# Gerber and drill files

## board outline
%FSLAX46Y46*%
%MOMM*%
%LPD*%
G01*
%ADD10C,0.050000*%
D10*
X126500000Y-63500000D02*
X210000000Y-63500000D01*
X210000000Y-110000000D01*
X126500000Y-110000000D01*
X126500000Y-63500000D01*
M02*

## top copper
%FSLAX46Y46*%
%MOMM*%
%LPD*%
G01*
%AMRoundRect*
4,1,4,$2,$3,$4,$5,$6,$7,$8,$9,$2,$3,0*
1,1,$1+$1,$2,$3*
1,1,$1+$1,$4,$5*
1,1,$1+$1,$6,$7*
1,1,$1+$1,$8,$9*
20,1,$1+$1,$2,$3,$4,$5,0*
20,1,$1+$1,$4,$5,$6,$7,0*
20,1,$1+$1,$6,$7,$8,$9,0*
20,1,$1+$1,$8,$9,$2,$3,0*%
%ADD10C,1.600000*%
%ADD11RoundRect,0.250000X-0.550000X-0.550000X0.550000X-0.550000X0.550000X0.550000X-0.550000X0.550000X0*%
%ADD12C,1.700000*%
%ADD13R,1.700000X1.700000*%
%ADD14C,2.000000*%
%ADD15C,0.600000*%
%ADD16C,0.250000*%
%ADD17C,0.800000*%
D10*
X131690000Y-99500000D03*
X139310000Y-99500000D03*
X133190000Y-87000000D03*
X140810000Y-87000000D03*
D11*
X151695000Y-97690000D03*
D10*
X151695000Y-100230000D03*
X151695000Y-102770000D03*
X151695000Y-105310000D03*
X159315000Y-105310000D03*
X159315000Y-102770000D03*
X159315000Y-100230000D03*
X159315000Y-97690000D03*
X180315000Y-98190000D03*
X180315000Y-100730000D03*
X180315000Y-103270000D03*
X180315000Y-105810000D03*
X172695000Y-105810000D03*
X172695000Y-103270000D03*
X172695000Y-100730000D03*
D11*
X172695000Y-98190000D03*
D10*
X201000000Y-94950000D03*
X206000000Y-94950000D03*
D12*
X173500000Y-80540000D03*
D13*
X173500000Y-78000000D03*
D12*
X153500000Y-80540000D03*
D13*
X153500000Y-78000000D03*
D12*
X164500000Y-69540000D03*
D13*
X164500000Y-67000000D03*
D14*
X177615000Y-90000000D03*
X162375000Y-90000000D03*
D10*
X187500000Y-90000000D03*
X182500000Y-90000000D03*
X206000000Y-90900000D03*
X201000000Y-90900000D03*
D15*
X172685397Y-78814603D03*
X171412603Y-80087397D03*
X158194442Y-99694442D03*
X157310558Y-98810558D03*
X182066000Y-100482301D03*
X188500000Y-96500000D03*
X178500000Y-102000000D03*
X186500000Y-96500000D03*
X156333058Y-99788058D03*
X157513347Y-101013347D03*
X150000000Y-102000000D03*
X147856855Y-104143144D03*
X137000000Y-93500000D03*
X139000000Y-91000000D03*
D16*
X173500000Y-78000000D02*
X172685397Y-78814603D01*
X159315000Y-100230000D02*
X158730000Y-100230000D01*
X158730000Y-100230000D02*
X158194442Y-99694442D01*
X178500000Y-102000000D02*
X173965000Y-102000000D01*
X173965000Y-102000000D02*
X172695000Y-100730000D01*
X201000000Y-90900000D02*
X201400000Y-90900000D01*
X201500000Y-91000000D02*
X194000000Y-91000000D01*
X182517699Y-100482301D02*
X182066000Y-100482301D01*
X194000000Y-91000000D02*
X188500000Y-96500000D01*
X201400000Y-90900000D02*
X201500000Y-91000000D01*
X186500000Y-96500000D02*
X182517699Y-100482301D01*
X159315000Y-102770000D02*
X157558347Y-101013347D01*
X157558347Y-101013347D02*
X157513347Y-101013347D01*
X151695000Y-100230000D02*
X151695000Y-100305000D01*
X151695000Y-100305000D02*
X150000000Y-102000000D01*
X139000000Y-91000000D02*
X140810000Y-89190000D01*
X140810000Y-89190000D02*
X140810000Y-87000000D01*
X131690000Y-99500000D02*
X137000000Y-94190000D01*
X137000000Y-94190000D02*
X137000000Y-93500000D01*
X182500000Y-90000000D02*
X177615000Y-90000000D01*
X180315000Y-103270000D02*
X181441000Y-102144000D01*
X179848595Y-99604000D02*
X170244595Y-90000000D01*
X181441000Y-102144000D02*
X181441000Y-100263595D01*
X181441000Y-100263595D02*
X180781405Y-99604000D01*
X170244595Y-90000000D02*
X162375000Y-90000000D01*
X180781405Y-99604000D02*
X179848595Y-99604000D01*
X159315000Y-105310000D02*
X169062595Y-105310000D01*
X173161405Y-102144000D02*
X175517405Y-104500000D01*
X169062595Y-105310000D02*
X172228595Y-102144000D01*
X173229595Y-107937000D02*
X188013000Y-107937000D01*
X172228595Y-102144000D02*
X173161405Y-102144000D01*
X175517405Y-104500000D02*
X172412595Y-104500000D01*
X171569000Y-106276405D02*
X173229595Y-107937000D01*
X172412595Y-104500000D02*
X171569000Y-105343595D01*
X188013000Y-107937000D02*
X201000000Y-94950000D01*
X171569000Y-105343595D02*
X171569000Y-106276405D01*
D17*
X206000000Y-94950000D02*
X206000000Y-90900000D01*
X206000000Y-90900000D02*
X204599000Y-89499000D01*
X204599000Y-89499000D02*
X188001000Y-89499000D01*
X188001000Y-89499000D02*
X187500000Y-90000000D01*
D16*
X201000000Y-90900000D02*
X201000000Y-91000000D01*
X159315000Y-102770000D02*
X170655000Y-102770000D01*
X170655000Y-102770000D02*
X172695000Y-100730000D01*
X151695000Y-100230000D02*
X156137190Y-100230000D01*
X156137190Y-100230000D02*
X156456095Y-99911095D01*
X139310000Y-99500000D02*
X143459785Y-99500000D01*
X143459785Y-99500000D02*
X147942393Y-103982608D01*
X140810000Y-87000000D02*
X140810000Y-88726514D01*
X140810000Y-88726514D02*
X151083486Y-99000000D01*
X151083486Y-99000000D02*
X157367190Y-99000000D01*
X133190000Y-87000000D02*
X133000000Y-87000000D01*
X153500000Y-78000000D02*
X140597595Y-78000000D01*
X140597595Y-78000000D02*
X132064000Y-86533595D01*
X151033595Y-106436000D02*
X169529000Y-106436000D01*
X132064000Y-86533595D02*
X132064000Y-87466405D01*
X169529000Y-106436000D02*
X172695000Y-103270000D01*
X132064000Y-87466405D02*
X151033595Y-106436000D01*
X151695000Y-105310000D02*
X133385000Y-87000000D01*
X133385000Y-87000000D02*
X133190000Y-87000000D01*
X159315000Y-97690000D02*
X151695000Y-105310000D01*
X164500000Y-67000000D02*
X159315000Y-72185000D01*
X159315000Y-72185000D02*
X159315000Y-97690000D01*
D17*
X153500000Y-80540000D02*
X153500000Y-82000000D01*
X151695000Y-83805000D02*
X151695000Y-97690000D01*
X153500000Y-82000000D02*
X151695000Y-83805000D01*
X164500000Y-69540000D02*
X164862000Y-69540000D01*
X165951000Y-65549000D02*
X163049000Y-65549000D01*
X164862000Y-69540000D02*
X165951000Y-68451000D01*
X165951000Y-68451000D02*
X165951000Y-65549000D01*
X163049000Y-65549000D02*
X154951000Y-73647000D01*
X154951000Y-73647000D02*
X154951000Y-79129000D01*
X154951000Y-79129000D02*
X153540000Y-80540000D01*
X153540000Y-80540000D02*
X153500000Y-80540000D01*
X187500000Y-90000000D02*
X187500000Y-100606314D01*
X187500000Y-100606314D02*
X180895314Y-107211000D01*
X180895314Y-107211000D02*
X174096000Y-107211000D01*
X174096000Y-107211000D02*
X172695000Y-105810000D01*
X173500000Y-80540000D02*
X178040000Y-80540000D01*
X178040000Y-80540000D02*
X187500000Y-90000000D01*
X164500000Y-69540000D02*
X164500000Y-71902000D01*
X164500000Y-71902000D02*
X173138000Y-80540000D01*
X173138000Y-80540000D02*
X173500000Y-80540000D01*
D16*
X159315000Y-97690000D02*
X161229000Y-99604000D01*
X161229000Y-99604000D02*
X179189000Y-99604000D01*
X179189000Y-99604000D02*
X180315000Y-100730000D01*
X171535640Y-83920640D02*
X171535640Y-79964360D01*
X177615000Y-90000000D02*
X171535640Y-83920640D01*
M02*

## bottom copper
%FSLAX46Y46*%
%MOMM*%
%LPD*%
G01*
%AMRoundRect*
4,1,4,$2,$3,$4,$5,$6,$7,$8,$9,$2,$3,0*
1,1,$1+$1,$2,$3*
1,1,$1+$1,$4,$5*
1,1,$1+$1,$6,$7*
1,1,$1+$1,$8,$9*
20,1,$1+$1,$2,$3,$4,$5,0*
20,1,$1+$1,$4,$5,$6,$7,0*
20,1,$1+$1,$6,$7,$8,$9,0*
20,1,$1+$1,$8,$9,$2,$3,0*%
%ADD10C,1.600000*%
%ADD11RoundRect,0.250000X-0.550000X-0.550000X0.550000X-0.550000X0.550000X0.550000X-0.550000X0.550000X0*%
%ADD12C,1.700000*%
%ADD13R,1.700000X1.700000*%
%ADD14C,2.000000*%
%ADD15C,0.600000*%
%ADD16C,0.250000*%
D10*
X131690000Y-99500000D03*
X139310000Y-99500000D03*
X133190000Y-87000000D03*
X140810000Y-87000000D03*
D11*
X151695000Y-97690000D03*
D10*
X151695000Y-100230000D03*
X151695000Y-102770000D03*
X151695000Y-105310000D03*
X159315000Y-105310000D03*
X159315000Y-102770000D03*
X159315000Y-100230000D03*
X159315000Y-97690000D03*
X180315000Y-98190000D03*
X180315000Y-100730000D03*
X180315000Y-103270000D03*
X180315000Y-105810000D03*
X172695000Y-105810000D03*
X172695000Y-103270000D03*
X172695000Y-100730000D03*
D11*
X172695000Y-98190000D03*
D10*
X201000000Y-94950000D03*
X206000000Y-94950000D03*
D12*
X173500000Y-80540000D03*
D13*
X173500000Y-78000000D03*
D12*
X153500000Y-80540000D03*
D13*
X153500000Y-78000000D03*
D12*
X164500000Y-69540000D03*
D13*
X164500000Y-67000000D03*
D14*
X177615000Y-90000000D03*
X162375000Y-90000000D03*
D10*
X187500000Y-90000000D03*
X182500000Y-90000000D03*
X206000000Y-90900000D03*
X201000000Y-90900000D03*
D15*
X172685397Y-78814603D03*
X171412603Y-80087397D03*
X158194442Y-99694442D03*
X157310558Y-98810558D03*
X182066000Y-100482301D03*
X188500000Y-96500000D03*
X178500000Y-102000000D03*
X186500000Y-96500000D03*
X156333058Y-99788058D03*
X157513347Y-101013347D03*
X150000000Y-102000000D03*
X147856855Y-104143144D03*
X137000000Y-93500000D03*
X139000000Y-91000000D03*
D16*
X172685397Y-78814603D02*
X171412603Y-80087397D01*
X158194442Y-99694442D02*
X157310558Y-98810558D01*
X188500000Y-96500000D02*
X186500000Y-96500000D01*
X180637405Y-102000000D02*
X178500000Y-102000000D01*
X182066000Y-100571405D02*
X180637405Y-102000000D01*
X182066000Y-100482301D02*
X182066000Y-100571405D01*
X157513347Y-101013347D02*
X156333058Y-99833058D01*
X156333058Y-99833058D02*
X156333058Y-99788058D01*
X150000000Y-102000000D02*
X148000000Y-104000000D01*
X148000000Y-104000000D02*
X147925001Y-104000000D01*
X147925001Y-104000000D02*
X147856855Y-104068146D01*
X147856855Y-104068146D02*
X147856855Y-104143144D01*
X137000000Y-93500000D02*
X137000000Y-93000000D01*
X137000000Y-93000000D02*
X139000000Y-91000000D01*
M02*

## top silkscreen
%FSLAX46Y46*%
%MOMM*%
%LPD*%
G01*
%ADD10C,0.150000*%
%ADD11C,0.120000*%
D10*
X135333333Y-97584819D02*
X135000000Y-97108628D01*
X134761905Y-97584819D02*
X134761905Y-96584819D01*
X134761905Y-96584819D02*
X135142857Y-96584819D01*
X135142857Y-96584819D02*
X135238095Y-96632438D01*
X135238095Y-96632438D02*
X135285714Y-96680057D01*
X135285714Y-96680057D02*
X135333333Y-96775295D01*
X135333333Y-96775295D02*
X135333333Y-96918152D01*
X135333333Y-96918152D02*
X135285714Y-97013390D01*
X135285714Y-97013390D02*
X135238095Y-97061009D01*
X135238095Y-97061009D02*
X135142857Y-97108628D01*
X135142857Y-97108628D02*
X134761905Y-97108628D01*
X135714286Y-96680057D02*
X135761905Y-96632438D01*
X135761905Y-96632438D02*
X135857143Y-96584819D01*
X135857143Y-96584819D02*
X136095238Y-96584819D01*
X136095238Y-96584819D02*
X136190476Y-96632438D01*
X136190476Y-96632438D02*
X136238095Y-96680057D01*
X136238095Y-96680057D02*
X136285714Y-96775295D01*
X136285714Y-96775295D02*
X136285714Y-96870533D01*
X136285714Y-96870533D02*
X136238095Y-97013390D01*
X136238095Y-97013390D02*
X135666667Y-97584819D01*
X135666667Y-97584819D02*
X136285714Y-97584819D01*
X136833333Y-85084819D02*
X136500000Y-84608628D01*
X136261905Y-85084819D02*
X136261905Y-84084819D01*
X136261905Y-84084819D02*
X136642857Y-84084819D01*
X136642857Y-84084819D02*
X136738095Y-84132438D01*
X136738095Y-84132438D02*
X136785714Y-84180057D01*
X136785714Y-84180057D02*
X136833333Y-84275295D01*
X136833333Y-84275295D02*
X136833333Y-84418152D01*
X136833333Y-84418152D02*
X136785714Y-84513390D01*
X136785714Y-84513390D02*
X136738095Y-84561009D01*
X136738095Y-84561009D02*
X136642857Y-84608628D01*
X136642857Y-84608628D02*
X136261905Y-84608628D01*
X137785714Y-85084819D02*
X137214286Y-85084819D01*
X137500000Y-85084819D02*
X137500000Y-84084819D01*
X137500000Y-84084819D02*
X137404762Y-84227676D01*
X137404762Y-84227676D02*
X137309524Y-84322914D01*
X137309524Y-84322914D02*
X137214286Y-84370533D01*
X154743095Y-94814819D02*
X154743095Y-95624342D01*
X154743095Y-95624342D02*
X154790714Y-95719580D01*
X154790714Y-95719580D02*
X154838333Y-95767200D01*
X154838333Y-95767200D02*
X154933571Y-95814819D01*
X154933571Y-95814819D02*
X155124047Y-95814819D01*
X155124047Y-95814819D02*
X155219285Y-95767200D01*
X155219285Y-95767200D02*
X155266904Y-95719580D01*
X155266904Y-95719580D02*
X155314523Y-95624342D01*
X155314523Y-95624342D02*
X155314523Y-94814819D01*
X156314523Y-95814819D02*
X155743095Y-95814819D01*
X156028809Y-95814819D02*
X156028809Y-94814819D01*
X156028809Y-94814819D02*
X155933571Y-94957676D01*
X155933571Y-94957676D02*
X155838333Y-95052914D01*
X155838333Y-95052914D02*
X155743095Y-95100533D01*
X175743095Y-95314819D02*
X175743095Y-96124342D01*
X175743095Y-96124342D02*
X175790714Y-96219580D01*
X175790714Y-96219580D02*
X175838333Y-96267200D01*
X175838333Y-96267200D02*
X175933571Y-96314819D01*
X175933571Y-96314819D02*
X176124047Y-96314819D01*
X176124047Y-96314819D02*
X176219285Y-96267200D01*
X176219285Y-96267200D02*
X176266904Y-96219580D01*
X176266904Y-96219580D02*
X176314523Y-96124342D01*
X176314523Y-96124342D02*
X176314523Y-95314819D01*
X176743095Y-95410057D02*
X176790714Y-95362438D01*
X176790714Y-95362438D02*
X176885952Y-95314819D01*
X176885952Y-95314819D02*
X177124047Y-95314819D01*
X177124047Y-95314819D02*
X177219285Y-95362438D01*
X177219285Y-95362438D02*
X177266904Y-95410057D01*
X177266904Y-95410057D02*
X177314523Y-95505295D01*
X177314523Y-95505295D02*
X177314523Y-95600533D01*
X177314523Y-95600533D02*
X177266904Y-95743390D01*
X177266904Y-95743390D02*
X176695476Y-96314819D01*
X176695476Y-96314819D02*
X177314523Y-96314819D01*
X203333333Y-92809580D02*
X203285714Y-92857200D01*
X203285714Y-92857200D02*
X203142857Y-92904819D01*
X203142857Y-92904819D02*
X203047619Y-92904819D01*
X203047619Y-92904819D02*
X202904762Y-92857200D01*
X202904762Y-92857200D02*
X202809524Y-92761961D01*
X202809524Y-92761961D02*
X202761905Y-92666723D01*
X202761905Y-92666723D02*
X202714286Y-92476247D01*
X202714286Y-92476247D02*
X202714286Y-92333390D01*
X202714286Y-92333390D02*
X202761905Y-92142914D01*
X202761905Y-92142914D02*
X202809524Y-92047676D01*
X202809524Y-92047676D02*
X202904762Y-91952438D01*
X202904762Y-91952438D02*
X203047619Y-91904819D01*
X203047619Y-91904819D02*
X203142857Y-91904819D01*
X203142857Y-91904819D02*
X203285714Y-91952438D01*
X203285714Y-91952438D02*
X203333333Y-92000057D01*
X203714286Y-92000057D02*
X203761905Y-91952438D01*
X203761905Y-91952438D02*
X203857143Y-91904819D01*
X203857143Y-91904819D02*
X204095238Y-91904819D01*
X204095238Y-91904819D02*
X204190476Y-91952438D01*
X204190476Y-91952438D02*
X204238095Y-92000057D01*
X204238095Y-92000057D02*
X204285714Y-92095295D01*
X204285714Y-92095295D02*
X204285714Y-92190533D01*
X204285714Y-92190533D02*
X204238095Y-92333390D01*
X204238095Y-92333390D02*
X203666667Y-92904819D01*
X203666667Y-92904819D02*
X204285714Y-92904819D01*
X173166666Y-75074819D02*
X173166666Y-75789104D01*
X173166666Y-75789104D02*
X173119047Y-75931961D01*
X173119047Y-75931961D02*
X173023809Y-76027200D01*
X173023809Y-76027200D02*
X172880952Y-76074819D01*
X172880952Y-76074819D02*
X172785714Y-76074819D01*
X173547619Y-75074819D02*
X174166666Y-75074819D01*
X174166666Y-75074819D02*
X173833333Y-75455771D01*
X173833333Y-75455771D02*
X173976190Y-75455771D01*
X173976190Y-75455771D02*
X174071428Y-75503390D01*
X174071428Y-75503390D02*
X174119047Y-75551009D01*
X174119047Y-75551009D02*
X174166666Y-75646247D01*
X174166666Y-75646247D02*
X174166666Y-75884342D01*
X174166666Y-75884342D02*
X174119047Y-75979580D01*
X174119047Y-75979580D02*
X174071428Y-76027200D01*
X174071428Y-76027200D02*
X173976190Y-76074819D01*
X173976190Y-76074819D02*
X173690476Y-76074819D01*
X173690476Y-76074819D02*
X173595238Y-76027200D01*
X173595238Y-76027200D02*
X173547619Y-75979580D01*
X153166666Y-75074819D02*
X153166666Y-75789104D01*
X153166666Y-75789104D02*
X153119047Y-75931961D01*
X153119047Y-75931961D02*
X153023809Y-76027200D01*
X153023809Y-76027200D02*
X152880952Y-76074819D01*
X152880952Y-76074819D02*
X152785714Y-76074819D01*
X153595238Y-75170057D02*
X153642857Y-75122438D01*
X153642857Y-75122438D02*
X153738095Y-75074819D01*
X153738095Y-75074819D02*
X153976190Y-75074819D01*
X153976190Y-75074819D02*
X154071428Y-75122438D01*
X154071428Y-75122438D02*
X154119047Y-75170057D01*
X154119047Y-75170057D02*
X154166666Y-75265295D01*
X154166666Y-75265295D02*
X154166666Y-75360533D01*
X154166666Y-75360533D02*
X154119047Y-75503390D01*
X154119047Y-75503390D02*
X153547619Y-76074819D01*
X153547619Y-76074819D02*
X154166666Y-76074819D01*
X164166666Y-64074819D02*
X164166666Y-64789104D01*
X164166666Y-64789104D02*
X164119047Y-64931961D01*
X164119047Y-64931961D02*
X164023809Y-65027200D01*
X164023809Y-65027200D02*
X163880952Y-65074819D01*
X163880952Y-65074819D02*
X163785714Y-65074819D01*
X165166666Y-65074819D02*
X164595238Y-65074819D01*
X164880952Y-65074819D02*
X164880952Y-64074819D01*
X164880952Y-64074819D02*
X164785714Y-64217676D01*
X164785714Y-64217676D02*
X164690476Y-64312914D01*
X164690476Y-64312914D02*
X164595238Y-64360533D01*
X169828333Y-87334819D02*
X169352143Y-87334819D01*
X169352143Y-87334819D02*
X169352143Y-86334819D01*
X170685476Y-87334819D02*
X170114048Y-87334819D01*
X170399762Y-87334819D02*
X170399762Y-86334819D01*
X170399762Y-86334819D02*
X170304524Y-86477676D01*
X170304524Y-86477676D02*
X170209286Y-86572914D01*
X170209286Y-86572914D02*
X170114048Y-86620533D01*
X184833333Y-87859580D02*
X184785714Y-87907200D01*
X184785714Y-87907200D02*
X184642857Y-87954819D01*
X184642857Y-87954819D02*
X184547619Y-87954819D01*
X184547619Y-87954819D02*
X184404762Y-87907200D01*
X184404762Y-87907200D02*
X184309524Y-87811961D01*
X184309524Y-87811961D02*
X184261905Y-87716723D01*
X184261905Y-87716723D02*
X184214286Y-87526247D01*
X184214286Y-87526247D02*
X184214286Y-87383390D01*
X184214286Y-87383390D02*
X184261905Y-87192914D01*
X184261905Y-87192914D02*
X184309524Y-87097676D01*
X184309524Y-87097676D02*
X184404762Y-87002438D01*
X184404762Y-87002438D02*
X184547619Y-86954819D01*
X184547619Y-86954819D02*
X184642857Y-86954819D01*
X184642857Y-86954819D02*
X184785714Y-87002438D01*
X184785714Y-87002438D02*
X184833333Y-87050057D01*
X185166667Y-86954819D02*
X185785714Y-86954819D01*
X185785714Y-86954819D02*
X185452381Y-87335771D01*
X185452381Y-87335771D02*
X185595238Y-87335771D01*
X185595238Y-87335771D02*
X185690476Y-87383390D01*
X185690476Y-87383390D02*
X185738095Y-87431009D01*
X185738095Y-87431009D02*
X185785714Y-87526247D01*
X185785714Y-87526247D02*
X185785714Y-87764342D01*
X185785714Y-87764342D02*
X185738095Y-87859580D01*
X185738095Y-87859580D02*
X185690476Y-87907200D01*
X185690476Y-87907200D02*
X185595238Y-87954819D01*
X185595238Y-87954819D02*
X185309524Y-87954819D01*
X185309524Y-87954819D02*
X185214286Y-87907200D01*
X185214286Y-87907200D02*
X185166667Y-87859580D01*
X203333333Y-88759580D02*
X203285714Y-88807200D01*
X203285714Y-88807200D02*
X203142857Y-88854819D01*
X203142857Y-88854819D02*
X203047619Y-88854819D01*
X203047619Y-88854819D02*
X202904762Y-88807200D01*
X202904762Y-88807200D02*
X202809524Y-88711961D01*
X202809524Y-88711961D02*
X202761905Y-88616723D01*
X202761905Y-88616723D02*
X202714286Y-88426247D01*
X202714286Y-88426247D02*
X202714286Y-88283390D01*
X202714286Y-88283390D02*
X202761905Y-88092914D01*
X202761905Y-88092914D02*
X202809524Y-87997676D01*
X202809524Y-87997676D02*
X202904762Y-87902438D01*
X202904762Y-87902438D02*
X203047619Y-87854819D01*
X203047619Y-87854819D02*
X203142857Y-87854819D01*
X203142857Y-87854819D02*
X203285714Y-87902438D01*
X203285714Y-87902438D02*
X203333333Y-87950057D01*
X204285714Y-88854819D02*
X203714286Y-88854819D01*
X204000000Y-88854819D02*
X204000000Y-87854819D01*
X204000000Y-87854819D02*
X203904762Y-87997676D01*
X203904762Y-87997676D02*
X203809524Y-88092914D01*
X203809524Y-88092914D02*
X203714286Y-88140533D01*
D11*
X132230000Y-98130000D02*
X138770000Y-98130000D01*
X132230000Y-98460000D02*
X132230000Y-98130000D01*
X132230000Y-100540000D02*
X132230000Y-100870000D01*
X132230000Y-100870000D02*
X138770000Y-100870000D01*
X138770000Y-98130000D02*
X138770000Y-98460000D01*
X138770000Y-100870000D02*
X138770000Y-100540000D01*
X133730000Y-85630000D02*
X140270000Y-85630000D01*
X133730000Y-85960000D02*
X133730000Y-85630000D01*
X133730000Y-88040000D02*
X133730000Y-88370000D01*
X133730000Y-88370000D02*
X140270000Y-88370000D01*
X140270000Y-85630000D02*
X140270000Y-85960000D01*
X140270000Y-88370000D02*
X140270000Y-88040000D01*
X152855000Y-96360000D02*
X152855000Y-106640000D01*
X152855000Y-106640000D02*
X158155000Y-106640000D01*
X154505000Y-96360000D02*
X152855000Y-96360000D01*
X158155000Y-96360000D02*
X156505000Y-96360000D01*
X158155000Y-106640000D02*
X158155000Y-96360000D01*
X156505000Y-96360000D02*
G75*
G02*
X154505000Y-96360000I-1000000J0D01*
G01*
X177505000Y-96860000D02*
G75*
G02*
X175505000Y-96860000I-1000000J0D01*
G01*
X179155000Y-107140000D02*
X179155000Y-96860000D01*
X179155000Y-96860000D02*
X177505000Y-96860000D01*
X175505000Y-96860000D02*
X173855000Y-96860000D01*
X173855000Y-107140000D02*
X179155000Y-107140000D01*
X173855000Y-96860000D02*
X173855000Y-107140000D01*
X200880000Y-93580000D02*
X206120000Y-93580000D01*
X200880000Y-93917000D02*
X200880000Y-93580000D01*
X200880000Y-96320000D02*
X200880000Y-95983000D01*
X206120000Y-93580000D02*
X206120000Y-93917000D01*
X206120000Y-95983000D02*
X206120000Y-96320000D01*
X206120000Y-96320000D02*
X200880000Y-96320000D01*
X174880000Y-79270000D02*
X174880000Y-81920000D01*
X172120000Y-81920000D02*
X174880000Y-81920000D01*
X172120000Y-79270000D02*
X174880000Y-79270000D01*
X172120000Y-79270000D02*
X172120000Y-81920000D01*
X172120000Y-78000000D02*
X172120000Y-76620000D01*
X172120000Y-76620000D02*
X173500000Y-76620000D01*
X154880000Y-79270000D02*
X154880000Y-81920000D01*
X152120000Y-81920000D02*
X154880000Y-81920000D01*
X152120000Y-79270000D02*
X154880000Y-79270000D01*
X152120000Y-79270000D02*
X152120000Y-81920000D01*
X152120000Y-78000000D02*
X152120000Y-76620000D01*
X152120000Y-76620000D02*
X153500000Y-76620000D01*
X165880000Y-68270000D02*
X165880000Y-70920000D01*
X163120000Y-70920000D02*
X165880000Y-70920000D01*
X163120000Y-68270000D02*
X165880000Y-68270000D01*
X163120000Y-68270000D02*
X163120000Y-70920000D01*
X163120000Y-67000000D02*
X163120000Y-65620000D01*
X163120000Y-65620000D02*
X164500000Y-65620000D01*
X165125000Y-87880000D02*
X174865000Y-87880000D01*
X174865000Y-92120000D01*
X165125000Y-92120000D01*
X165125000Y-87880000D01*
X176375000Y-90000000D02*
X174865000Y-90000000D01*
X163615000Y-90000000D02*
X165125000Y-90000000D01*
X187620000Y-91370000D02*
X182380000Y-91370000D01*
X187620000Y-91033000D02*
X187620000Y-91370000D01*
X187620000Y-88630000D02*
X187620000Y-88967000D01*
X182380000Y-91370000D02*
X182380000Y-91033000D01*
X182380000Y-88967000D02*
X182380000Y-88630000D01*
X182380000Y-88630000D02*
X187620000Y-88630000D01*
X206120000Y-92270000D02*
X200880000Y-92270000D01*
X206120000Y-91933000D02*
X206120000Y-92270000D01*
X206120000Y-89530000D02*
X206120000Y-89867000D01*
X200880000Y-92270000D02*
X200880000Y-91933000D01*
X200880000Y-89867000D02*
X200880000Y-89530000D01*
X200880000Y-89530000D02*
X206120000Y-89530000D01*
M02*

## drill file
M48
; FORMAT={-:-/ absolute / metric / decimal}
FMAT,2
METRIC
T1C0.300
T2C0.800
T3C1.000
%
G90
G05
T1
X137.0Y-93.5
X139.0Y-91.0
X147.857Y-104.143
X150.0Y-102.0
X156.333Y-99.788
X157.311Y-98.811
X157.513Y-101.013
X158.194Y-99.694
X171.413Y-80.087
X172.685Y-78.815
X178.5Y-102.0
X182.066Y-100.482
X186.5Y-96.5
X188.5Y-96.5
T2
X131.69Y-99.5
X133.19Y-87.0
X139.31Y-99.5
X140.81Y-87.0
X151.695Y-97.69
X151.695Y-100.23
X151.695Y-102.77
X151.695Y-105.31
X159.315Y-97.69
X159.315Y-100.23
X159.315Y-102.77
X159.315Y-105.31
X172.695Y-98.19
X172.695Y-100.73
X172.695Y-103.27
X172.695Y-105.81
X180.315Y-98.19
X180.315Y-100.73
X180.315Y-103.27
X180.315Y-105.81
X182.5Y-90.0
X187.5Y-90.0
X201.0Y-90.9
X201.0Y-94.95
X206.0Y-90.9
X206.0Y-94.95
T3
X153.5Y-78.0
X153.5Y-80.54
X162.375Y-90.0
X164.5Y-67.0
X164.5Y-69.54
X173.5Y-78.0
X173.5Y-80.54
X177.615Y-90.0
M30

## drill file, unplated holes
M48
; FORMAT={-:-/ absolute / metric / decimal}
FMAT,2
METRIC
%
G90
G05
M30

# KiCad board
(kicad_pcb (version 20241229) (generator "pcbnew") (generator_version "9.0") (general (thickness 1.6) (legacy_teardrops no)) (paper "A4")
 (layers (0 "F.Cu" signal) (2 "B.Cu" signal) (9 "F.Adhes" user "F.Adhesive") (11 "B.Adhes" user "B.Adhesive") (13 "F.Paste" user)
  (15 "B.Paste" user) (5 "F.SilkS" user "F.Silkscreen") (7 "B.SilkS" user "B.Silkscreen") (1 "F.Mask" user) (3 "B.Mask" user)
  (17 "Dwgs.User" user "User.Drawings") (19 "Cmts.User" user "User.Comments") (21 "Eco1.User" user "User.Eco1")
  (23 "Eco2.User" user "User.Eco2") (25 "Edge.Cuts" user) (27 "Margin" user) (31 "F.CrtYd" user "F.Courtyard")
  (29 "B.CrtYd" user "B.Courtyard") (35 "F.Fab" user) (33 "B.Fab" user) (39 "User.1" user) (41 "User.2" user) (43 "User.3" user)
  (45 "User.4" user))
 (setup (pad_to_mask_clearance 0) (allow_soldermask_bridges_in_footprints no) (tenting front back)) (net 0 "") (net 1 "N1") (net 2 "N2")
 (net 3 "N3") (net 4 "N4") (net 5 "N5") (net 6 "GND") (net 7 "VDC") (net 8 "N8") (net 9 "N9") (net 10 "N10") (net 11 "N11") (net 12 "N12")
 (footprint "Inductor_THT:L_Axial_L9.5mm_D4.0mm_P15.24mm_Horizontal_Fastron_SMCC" (layer "F.Cu") (at 162.375 90)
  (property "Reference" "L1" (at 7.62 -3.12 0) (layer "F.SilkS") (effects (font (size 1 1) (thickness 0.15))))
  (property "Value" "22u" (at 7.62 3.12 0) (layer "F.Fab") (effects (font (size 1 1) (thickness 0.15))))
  (fp_line (start 1.24 0) (end 2.75 0) (stroke (width 0.12) (type solid)) (layer "F.SilkS"))
  (fp_line (start 14 0) (end 12.49 0) (stroke (width 0.12) (type solid)) (layer "F.SilkS"))
  (fp_rect (start 2.75 -2.12) (end 12.49 2.12) (stroke (width 0.12) (type solid)) (fill no) (layer "F.SilkS"))
  (pad "1" thru_hole circle (at 0 0) (size 2 2) (drill 1) (layers "*.Cu" "*.Mask") (remove_unused_layers no) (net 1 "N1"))
  (pad "2" thru_hole circle (at 15.24 0) (size 2 2) (drill 1) (layers "*.Cu" "*.Mask") (remove_unused_layers no) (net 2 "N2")))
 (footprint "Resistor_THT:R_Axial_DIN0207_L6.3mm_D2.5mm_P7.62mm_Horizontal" (layer "F.Cu") (at 131.69 99.5)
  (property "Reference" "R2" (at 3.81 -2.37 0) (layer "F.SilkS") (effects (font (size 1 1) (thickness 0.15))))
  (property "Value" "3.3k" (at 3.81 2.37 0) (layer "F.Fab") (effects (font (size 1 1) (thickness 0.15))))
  (fp_line (start 0.54 -1.37) (end 7.08 -1.37) (stroke (width 0.12) (type solid)) (layer "F.SilkS"))
  (fp_line (start 0.54 -1.04) (end 0.54 -1.37) (stroke (width 0.12) (type solid)) (layer "F.SilkS"))
  (fp_line (start 0.54 1.04) (end 0.54 1.37) (stroke (width 0.12) (type solid)) (layer "F.SilkS"))
  (fp_line (start 0.54 1.37) (end 7.08 1.37) (stroke (width 0.12) (type solid)) (layer "F.SilkS"))
  (fp_line (start 7.08 -1.37) (end 7.08 -1.04) (stroke (width 0.12) (type solid)) (layer "F.SilkS"))
  (fp_line (start 7.08 1.37) (end 7.08 1.04) (stroke (width 0.12) (type solid)) (layer "F.SilkS"))
  (pad "1" thru_hole circle (at 0 0) (size 1.6 1.6) (drill 0.8) (layers "*.Cu" "*.Mask") (remove_unused_layers no) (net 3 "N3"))
  (pad "2" thru_hole circle (at 7.62 0) (size 1.6 1.6) (drill 0.8) (layers "*.Cu" "*.Mask") (remove_unused_layers no) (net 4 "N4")))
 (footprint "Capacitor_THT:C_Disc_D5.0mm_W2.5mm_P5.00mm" (layer "F.Cu") (at 201 94.95)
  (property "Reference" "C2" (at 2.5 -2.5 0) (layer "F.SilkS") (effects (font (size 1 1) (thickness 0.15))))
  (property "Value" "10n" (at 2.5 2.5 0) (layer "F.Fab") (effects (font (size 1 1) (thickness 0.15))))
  (fp_line (start -0.12 -1.37) (end 5.12 -1.37) (stroke (width 0.12) (type solid)) (layer "F.SilkS"))
  (fp_line (start -0.12 -1.033) (end -0.12 -1.37) (stroke (width 0.12) (type solid)) (layer "F.SilkS"))
  (fp_line (start -0.12 1.37) (end -0.12 1.033) (stroke (width 0.12) (type solid)) (layer "F.SilkS"))
  (fp_line (start 5.12 -1.37) (end 5.12 -1.033) (stroke (width 0.12) (type solid)) (layer "F.SilkS"))
  (fp_line (start 5.12 1.033) (end 5.12 1.37) (stroke (width 0.12) (type solid)) (layer "F.SilkS"))
  (fp_line (start 5.12 1.37) (end -0.12 1.37) (stroke (width 0.12) (type solid)) (layer "F.SilkS"))
  (pad "1" thru_hole circle (at 0 0) (size 1.6 1.6) (drill 0.8) (layers "*.Cu" "*.Mask") (remove_unused_layers no) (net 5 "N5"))
  (pad "2" thru_hole circle (at 5 0) (size 1.6 1.6) (drill 0.8) (layers "*.Cu" "*.Mask") (remove_unused_layers no) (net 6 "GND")))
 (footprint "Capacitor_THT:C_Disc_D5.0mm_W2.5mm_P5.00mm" (layer "F.Cu") (at 182.5 90)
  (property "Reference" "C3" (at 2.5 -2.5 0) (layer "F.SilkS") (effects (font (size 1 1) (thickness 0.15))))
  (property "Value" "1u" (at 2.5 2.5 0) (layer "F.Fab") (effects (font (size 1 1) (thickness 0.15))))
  (fp_line (start -0.12 -1.37) (end 5.12 -1.37) (stroke (width 0.12) (type solid)) (layer "F.SilkS"))
  (fp_line (start -0.12 -1.033) (end -0.12 -1.37) (stroke (width 0.12) (type solid)) (layer "F.SilkS"))
  (fp_line (start -0.12 1.37) (end -0.12 1.033) (stroke (width 0.12) (type solid)) (layer "F.SilkS"))
  (fp_line (start 5.12 -1.37) (end 5.12 -1.033) (stroke (width 0.12) (type solid)) (layer "F.SilkS"))
  (fp_line (start 5.12 1.033) (end 5.12 1.37) (stroke (width 0.12) (type solid)) (layer "F.SilkS"))
  (fp_line (start 5.12 1.37) (end -0.12 1.37) (stroke (width 0.12) (type solid)) (layer "F.SilkS"))
  (pad "1" thru_hole circle (at 0 0) (size 1.6 1.6) (drill 0.8) (layers "*.Cu" "*.Mask") (remove_unused_layers no) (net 2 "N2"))
  (pad "2" thru_hole circle (at 5 0) (size 1.6 1.6) (drill 0.8) (layers "*.Cu" "*.Mask") (remove_unused_layers no) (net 6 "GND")))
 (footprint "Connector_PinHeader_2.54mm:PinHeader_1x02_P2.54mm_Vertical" (layer "F.Cu") (at 164.5 67)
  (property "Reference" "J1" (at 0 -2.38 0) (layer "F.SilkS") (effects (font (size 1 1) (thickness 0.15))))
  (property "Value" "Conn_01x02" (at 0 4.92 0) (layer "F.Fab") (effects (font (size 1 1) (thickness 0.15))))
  (fp_line (start -1.38 -1.38) (end 0 -1.38) (stroke (width 0.12) (type solid)) (layer "F.SilkS"))
  (fp_line (start -1.38 0) (end -1.38 -1.38) (stroke (width 0.12) (type solid)) (layer "F.SilkS"))
  (fp_line (start -1.38 1.27) (end -1.38 3.92) (stroke (width 0.12) (type solid)) (layer "F.SilkS"))
  (fp_line (start -1.38 1.27) (end 1.38 1.27) (stroke (width 0.12) (type solid)) (layer "F.SilkS"))
  (fp_line (start -1.38 3.92) (end 1.38 3.92) (stroke (width 0.12) (type solid)) (layer "F.SilkS"))
  (fp_line (start 1.38 1.27) (end 1.38 3.92) (stroke (width 0.12) (type solid)) (layer "F.SilkS"))
  (pad "1" thru_hole rect (at 0 0) (size 1.7 1.7) (drill 1) (layers "*.Cu" "*.Mask") (remove_unused_layers no) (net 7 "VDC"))
  (pad "2" thru_hole circle (at 0 2.54) (size 1.7 1.7) (drill 1) (layers "*.Cu" "*.Mask") (remove_unused_layers no) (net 6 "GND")))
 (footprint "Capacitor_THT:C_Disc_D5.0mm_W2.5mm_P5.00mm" (layer "F.Cu") (at 201 90.9)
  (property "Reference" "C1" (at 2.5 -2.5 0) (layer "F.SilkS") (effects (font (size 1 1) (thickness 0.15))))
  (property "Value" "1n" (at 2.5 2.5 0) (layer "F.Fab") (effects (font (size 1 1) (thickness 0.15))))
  (fp_line (start -0.12 -1.37) (end 5.12 -1.37) (stroke (width 0.12) (type solid)) (layer "F.SilkS"))
  (fp_line (start -0.12 -1.033) (end -0.12 -1.37) (stroke (width 0.12) (type solid)) (layer "F.SilkS"))
  (fp_line (start -0.12 1.37) (end -0.12 1.033) (stroke (width 0.12) (type solid)) (layer "F.SilkS"))
  (fp_line (start 5.12 -1.37) (end 5.12 -1.033) (stroke (width 0.12) (type solid)) (layer "F.SilkS"))
  (fp_line (start 5.12 1.033) (end 5.12 1.37) (stroke (width 0.12) (type solid)) (layer "F.SilkS"))
  (fp_line (start 5.12 1.37) (end -0.12 1.37) (stroke (width 0.12) (type solid)) (layer "F.SilkS"))
  (pad "1" thru_hole circle (at 0 0) (size 1.6 1.6) (drill 0.8) (layers "*.Cu" "*.Mask") (remove_unused_layers no) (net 4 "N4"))
  (pad "2" thru_hole circle (at 5 0) (size 1.6 1.6) (drill 0.8) (layers "*.Cu" "*.Mask") (remove_unused_layers no) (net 6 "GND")))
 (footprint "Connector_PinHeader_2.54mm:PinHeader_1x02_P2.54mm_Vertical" (layer "F.Cu") (at 153.5 78)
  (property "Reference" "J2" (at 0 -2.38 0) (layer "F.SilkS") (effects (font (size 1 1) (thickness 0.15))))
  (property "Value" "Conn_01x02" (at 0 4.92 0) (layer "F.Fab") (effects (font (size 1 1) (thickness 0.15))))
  (fp_line (start -1.38 -1.38) (end 0 -1.38) (stroke (width 0.12) (type solid)) (layer "F.SilkS"))
  (fp_line (start -1.38 0) (end -1.38 -1.38) (stroke (width 0.12) (type solid)) (layer "F.SilkS"))
  (fp_line (start -1.38 1.27) (end -1.38 3.92) (stroke (width 0.12) (type solid)) (layer "F.SilkS"))
  (fp_line (start -1.38 1.27) (end 1.38 1.27) (stroke (width 0.12) (type solid)) (layer "F.SilkS"))
  (fp_line (start -1.38 3.92) (end 1.38 3.92) (stroke (width 0.12) (type solid)) (layer "F.SilkS"))
  (fp_line (start 1.38 1.27) (end 1.38 3.92) (stroke (width 0.12) (type solid)) (layer "F.SilkS"))
  (pad "1" thru_hole rect (at 0 0) (size 1.7 1.7) (drill 1) (layers "*.Cu" "*.Mask") (remove_unused_layers no) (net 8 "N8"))
  (pad "2" thru_hole circle (at 0 2.54) (size 1.7 1.7) (drill 1) (layers "*.Cu" "*.Mask") (remove_unused_layers no) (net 6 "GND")))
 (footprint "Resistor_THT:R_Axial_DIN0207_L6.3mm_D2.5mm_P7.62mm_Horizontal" (layer "F.Cu") (at 133.19 87)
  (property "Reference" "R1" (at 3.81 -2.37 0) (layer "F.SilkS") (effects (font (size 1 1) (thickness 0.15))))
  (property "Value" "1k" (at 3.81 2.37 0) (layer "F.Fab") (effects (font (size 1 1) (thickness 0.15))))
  (fp_line (start 0.54 -1.37) (end 7.08 -1.37) (stroke (width 0.12) (type solid)) (layer "F.SilkS"))
  (fp_line (start 0.54 -1.04) (end 0.54 -1.37) (stroke (width 0.12) (type solid)) (layer "F.SilkS"))
  (fp_line (start 0.54 1.04) (end 0.54 1.37) (stroke (width 0.12) (type solid)) (layer "F.SilkS"))
  (fp_line (start 0.54 1.37) (end 7.08 1.37) (stroke (width 0.12) (type solid)) (layer "F.SilkS"))
  (fp_line (start 7.08 -1.37) (end 7.08 -1.04) (stroke (width 0.12) (type solid)) (layer "F.SilkS"))
  (fp_line (start 7.08 1.37) (end 7.08 1.04) (stroke (width 0.12) (type solid)) (layer "F.SilkS"))
  (pad "1" thru_hole circle (at 0 0) (size 1.6 1.6) (drill 0.8) (layers "*.Cu" "*.Mask") (remove_unused_layers no) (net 7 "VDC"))
  (pad "2" thru_hole circle (at 7.62 0) (size 1.6 1.6) (drill 0.8) (layers "*.Cu" "*.Mask") (remove_unused_layers no) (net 3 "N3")))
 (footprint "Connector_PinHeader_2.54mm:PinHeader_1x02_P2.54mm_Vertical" (layer "F.Cu") (at 173.5 78)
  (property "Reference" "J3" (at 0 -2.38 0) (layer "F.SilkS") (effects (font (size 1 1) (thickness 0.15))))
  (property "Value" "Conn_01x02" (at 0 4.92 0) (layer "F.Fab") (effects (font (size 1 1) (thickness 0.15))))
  (fp_line (start -1.38 -1.38) (end 0 -1.38) (stroke (width 0.12) (type solid)) (layer "F.SilkS"))
  (fp_line (start -1.38 0) (end -1.38 -1.38) (stroke (width 0.12) (type solid)) (layer "F.SilkS"))
  (fp_line (start -1.38 1.27) (end -1.38 3.92) (stroke (width 0.12) (type solid)) (layer "F.SilkS"))
  (fp_line (start -1.38 1.27) (end 1.38 1.27) (stroke (width 0.12) (type solid)) (layer "F.SilkS"))
  (fp_line (start -1.38 3.92) (end 1.38 3.92) (stroke (width 0.12) (type solid)) (layer "F.SilkS"))
  (fp_line (start 1.38 1.27) (end 1.38 3.92) (stroke (width 0.12) (type solid)) (layer "F.SilkS"))
  (pad "1" thru_hole rect (at 0 0) (size 1.7 1.7) (drill 1) (layers "*.Cu" "*.Mask") (remove_unused_layers no) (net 2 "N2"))
  (pad "2" thru_hole circle (at 0 2.54) (size 1.7 1.7) (drill 1) (layers "*.Cu" "*.Mask") (remove_unused_layers no) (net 6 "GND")))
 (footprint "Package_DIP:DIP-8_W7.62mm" (layer "F.Cu") (at 172.695 98.19)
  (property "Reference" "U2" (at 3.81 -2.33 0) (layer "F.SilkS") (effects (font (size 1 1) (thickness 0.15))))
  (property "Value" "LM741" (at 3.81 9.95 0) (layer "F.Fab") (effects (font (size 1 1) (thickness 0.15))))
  (fp_line (start 1.16 -1.33) (end 1.16 8.95) (stroke (width 0.12) (type solid)) (layer "F.SilkS"))
  (fp_line (start 1.16 8.95) (end 6.46 8.95) (stroke (width 0.12) (type solid)) (layer "F.SilkS"))
  (fp_line (start 2.81 -1.33) (end 1.16 -1.33) (stroke (width 0.12) (type solid)) (layer "F.SilkS"))
  (fp_line (start 6.46 -1.33) (end 4.81 -1.33) (stroke (width 0.12) (type solid)) (layer "F.SilkS"))
  (fp_line (start 6.46 8.95) (end 6.46 -1.33) (stroke (width 0.12) (type solid)) (layer "F.SilkS"))
  (fp_arc (start 4.81 -1.33) (mid 3.81 -0.33) (end 2.81 -1.33) (stroke (width 0.12) (type solid)) (layer "F.SilkS"))
  (pad "1" thru_hole roundrect (at 0 0) (size 1.6 1.6) (drill 0.8) (layers "*.Cu" "*.Mask") (remove_unused_layers no)
   (roundrect_rratio 0.15625) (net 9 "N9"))
  (pad "2" thru_hole circle (at 0 2.54) (size 1.6 1.6) (drill 0.8) (layers "*.Cu" "*.Mask") (remove_unused_layers no) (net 4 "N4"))
  (pad "3" thru_hole circle (at 0 5.08) (size 1.6 1.6) (drill 0.8) (layers "*.Cu" "*.Mask") (remove_unused_layers no) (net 8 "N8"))
  (pad "4" thru_hole circle (at 0 7.62) (size 1.6 1.6) (drill 0.8) (layers "*.Cu" "*.Mask") (remove_unused_layers no) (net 6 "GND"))
  (pad "5" thru_hole circle (at 7.62 7.62) (size 1.6 1.6) (drill 0.8) (layers "*.Cu" "*.Mask") (remove_unused_layers no) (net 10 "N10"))
  (pad "6" thru_hole circle (at 7.62 5.08) (size 1.6 1.6) (drill 0.8) (layers "*.Cu" "*.Mask") (remove_unused_layers no) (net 1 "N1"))
  (pad "7" thru_hole circle (at 7.62 2.54) (size 1.6 1.6) (drill 0.8) (layers "*.Cu" "*.Mask") (remove_unused_layers no) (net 7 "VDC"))
  (pad "8" thru_hole circle (at 7.62 0) (size 1.6 1.6) (drill 0.8) (layers "*.Cu" "*.Mask") (remove_unused_layers no) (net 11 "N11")))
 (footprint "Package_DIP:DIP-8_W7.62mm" (layer "F.Cu") (at 151.695 97.69)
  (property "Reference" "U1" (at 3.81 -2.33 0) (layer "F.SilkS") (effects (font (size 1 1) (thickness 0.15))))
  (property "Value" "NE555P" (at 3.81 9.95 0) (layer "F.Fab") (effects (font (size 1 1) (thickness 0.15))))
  (fp_line (start 1.16 -1.33) (end 1.16 8.95) (stroke (width 0.12) (type solid)) (layer "F.SilkS"))
  (fp_line (start 1.16 8.95) (end 6.46 8.95) (stroke (width 0.12) (type solid)) (layer "F.SilkS"))
  (fp_line (start 2.81 -1.33) (end 1.16 -1.33) (stroke (width 0.12) (type solid)) (layer "F.SilkS"))
  (fp_line (start 6.46 -1.33) (end 4.81 -1.33) (stroke (width 0.12) (type solid)) (layer "F.SilkS"))
  (fp_line (start 6.46 8.95) (end 6.46 -1.33) (stroke (width 0.12) (type solid)) (layer "F.SilkS"))
  (fp_arc (start 4.81 -1.33) (mid 3.81 -0.33) (end 2.81 -1.33) (stroke (width 0.12) (type solid)) (layer "F.SilkS"))
  (pad "1" thru_hole roundrect (at 0 0) (size 1.6 1.6) (drill 0.8) (layers "*.Cu" "*.Mask") (remove_unused_layers no)
   (roundrect_rratio 0.15625) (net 6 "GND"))
  (pad "2" thru_hole circle (at 0 2.54) (size 1.6 1.6) (drill 0.8) (layers "*.Cu" "*.Mask") (remove_unused_layers no) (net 4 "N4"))
  (pad "3" thru_hole circle (at 0 5.08) (size 1.6 1.6) (drill 0.8) (layers "*.Cu" "*.Mask") (remove_unused_layers no) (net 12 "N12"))
  (pad "4" thru_hole circle (at 0 7.62) (size 1.6 1.6) (drill 0.8) (layers "*.Cu" "*.Mask") (remove_unused_layers no) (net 7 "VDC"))
  (pad "5" thru_hole circle (at 7.62 7.62) (size 1.6 1.6) (drill 0.8) (layers "*.Cu" "*.Mask") (remove_unused_layers no) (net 5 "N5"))
  (pad "6" thru_hole circle (at 7.62 5.08) (size 1.6 1.6) (drill 0.8) (layers "*.Cu" "*.Mask") (remove_unused_layers no) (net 4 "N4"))
  (pad "7" thru_hole circle (at 7.62 2.54) (size 1.6 1.6) (drill 0.8) (layers "*.Cu" "*.Mask") (remove_unused_layers no) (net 3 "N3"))
  (pad "8" thru_hole circle (at 7.62 0) (size 1.6 1.6) (drill 0.8) (layers "*.Cu" "*.Mask") (remove_unused_layers no) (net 7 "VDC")))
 (gr_rect (start 126.5 63.5) (end 210 110) (stroke (width 0.05) (type default)) (fill no) (layer "Edge.Cuts"))
 (segment (start 153.5 82) (end 151.695 83.805) (width 0.8) (layer "F.Cu") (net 6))
 (segment (start 188.001 89.499) (end 187.5 90) (width 0.8) (layer "F.Cu") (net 6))
 (segment (start 173.138 80.54) (end 173.5 80.54) (width 0.8) (layer "F.Cu") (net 6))
 (segment (start 180.895314 107.211) (end 174.096 107.211) (width 0.8) (layer "F.Cu") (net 6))
 (segment (start 153.54 80.54) (end 153.5 80.54) (width 0.8) (layer "F.Cu") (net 6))
 (segment (start 163.049 65.549) (end 154.951 73.647) (width 0.8) (layer "F.Cu") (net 6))
 (segment (start 153.5 80.54) (end 153.5 82) (width 0.8) (layer "F.Cu") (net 6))
 (segment (start 164.862 69.54) (end 165.951 68.451) (width 0.8) (layer "F.Cu") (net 6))
 (segment (start 164.5 69.54) (end 164.862 69.54) (width 0.8) (layer "F.Cu") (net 6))
 (segment (start 151.695 83.805) (end 151.695 97.69) (width 0.8) (layer "F.Cu") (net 6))
 (segment (start 164.5 69.54) (end 164.5 71.902) (width 0.8) (layer "F.Cu") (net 6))
 (segment (start 173.5 80.54) (end 178.04 80.54) (width 0.8) (layer "F.Cu") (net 6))
 (segment (start 178.04 80.54) (end 187.5 90) (width 0.8) (layer "F.Cu") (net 6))
 (segment (start 204.599 89.499) (end 188.001 89.499) (width 0.8) (layer "F.Cu") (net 6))
 (segment (start 154.951 79.129) (end 153.54 80.54) (width 0.8) (layer "F.Cu") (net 6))
 (segment (start 154.951 73.647) (end 154.951 79.129) (width 0.8) (layer "F.Cu") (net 6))
 (segment (start 187.5 100.606314) (end 180.895314 107.211) (width 0.8) (layer "F.Cu") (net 6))
 (segment (start 206 94.95) (end 206 90.9) (width 0.8) (layer "F.Cu") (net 6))
 (segment (start 165.951 68.451) (end 165.951 65.549) (width 0.8) (layer "F.Cu") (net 6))
 (segment (start 174.096 107.211) (end 172.695 105.81) (width 0.8) (layer "F.Cu") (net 6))
 (segment (start 164.5 71.902) (end 173.138 80.54) (width 0.8) (layer "F.Cu") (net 6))
 (segment (start 187.5 90) (end 187.5 100.606314) (width 0.8) (layer "F.Cu") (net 6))
 (segment (start 206 90.9) (end 204.599 89.499) (width 0.8) (layer "F.Cu") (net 6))
 (segment (start 165.951 65.549) (end 163.049 65.549) (width 0.8) (layer "F.Cu") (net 6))
 (segment (start 194 91) (end 188.5 96.5) (width 0.25) (layer "F.Cu") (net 4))
 (segment (start 186.5 96.5) (end 182.517699 100.482301) (width 0.25) (layer "F.Cu") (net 4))
 (segment (start 151.695 100.23) (end 151.695 100.305) (width 0.25) (layer "F.Cu") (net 4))
 (segment (start 151.695 100.305) (end 150 102) (width 0.25) (layer "F.Cu") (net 4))
 (segment (start 201 90.9) (end 201.4 90.9) (width 0.25) (layer "F.Cu") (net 4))
 (segment (start 170.655 102.77) (end 172.695 100.73) (width 0.25) (layer "F.Cu") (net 4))
 (segment (start 157.558347 101.013347) (end 157.513347 101.013347) (width 0.25) (layer "F.Cu") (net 4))
 (segment (start 159.315 102.77) (end 157.558347 101.013347) (width 0.25) (layer "F.Cu") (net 4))
 (segment (start 182.517699 100.482301) (end 182.066 100.482301) (width 0.25) (layer "F.Cu") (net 4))
 (segment (start 139.31 99.5) (end 143.459785 99.5) (width 0.25) (layer "F.Cu") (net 4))
 (segment (start 178.5 102) (end 173.965 102) (width 0.25) (layer "F.Cu") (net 4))
 (segment (start 201.4 90.9) (end 201.5 91) (width 0.25) (layer "F.Cu") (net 4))
 (segment (start 151.695 100.23) (end 156.13719 100.23) (width 0.25) (layer "F.Cu") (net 4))
 (segment (start 159.315 102.77) (end 170.655 102.77) (width 0.25) (layer "F.Cu") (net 4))
 (segment (start 201.5 91) (end 194 91) (width 0.25) (layer "F.Cu") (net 4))
 (segment (start 201 90.9) (end 201 91) (width 0.25) (layer "F.Cu") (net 4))
 (segment (start 173.965 102) (end 172.695 100.73) (width 0.25) (layer "F.Cu") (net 4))
 (segment (start 143.459785 99.5) (end 147.942393 103.982608) (width 0.25) (layer "F.Cu") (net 4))
 (segment (start 156.13719 100.23) (end 156.456095 99.911095) (width 0.25) (layer "F.Cu") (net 4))
 (via (at 150 102) (size 0.6) (drill 0.3) (layers "F.Cu" "B.Cu") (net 4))
 (via (at 157.513347 101.013347) (size 0.6) (drill 0.3) (layers "F.Cu" "B.Cu") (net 4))
 (via (at 156.333058 99.788058) (size 0.6) (drill 0.3) (layers "F.Cu" "B.Cu") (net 4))
 (via (at 147.856855 104.143144) (size 0.6) (drill 0.3) (layers "F.Cu" "B.Cu") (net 4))
 (via (at 186.5 96.5) (size 0.6) (drill 0.3) (layers "F.Cu" "B.Cu") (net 4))
 (via (at 182.066 100.482301) (size 0.6) (drill 0.3) (layers "F.Cu" "B.Cu") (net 4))
 (via (at 188.5 96.5) (size 0.6) (drill 0.3) (layers "F.Cu" "B.Cu") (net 4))
 (via (at 178.5 102) (size 0.6) (drill 0.3) (layers "F.Cu" "B.Cu") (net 4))
 (segment (start 156.333058 99.833058) (end 156.333058 99.788058) (width 0.25) (layer "B.Cu") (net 4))
 (segment (start 182.066 100.571405) (end 180.637405 102) (width 0.25) (layer "B.Cu") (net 4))
 (segment (start 148 104) (end 147.925001 104) (width 0.25) (layer "B.Cu") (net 4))
 (segment (start 150 102) (end 148 104) (width 0.25) (layer "B.Cu") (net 4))
 (segment (start 147.856855 104.068146) (end 147.856855 104.143144) (width 0.25) (layer "B.Cu") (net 4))
 (segment (start 157.513347 101.013347) (end 156.333058 99.833058) (width 0.25) (layer "B.Cu") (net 4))
 (segment (start 147.925001 104) (end 147.856855 104.068146) (width 0.25) (layer "B.Cu") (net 4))
 (segment (start 182.066 100.482301) (end 182.066 100.571405) (width 0.25) (layer "B.Cu") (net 4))
 (segment (start 188.5 96.5) (end 186.5 96.5) (width 0.25) (layer "B.Cu") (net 4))
 (segment (start 180.637405 102) (end 178.5 102) (width 0.25) (layer "B.Cu") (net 4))
 (segment (start 159.315 105.31) (end 169.062595 105.31) (width 0.25) (layer "F.Cu") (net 5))
 (segment (start 171.569 105.343595) (end 171.569 106.276405) (width 0.25) (layer "F.Cu") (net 5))
 (segment (start 173.161405 102.144) (end 175.517405 104.5) (width 0.25) (layer "F.Cu") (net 5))
 (segment (start 173.229595 107.937) (end 188.013 107.937) (width 0.25) (layer "F.Cu") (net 5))
 (segment (start 169.062595 105.31) (end 172.228595 102.144) (width 0.25) (layer "F.Cu") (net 5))
 (segment (start 172.228595 102.144) (end 173.161405 102.144) (width 0.25) (layer "F.Cu") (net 5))
 (segment (start 175.517405 104.5) (end 172.412595 104.5) (width 0.25) (layer "F.Cu") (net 5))
 (segment (start 188.013 107.937) (end 201 94.95) (width 0.25) (layer "F.Cu") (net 5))
 (segment (start 172.412595 104.5) (end 171.569 105.343595) (width 0.25) (layer "F.Cu") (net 5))
 (segment (start 171.569 106.276405) (end 173.229595 107.937) (width 0.25) (layer "F.Cu") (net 5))
 (segment (start 177.615 90) (end 171.53564 83.92064) (width 0.25) (layer "F.Cu") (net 2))
 (segment (start 171.53564 83.92064) (end 171.53564 79.96436) (width 0.25) (layer "F.Cu") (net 2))
 (segment (start 182.5 90) (end 177.615 90) (width 0.25) (layer "F.Cu") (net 2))
 (segment (start 173.5 78) (end 172.685397 78.814603) (width 0.25) (layer "F.Cu") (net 2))
 (via (at 172.685397 78.814603) (size 0.6) (drill 0.3) (layers "F.Cu" "B.Cu") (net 2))
 (via (at 171.412603 80.087397) (size 0.6) (drill 0.3) (layers "F.Cu" "B.Cu") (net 2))
 (segment (start 172.685397 78.814603) (end 171.412603 80.087397) (width 0.25) (layer "B.Cu") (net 2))
 (segment (start 151.695 105.31) (end 133.385 87) (width 0.25) (layer "F.Cu") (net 7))
 (segment (start 164.5 67) (end 159.315 72.185) (width 0.25) (layer "F.Cu") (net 7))
 (segment (start 159.315 97.69) (end 161.229 99.604) (width 0.25) (layer "F.Cu") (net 7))
 (segment (start 179.189 99.604) (end 180.315 100.73) (width 0.25) (layer "F.Cu") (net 7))
 (segment (start 159.315 72.185) (end 159.315 97.69) (width 0.25) (layer "F.Cu") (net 7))
 (segment (start 161.229 99.604) (end 179.189 99.604) (width 0.25) (layer "F.Cu") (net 7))
 (segment (start 133.385 87) (end 133.19 87) (width 0.25) (layer "F.Cu") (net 7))
 (segment (start 159.315 97.69) (end 151.695 105.31) (width 0.25) (layer "F.Cu") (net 7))
 (segment (start 133.19 87) (end 133 87) (width 0.25) (layer "F.Cu") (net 7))
 (segment (start 132.064 86.533595) (end 132.064 87.466405) (width 0.25) (layer "F.Cu") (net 8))
 (segment (start 151.033595 106.436) (end 169.529 106.436) (width 0.25) (layer "F.Cu") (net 8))
 (segment (start 132.064 87.466405) (end 151.033595 106.436) (width 0.25) (layer "F.Cu") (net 8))
 (segment (start 153.5 78) (end 140.597595 78) (width 0.25) (layer "F.Cu") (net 8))
 (segment (start 169.529 106.436) (end 172.695 103.27) (width 0.25) (layer "F.Cu") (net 8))
 (segment (start 140.597595 78) (end 132.064 86.533595) (width 0.25) (layer "F.Cu") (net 8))
 (segment (start 181.441 100.263595) (end 180.781405 99.604) (width 0.25) (layer "F.Cu") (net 1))
 (segment (start 170.244595 90) (end 162.375 90) (width 0.25) (layer "F.Cu") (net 1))
 (segment (start 180.781405 99.604) (end 179.848595 99.604) (width 0.25) (layer "F.Cu") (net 1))
 (segment (start 180.315 103.27) (end 181.441 102.144) (width 0.25) (layer "F.Cu") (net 1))
 (segment (start 179.848595 99.604) (end 170.244595 90) (width 0.25) (layer "F.Cu") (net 1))
 (segment (start 181.441 102.144) (end 181.441 100.263595) (width 0.25) (layer "F.Cu") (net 1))
 (segment (start 131.69 99.5) (end 137 94.19) (width 0.25) (layer "F.Cu") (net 3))
 (segment (start 140.81 88.726514) (end 151.083486 99) (width 0.25) (layer "F.Cu") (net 3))
 (segment (start 137 94.19) (end 137 93.5) (width 0.25) (layer "F.Cu") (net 3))
 (segment (start 151.083486 99) (end 157.36719 99) (width 0.25) (layer "F.Cu") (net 3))
 (segment (start 140.81 89.19) (end 140.81 87) (width 0.25) (layer "F.Cu") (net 3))
 (segment (start 158.73 100.23) (end 158.194442 99.694442) (width 0.25) (layer "F.Cu") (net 3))
 (segment (start 139 91) (end 140.81 89.19) (width 0.25) (layer "F.Cu") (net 3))
 (segment (start 140.81 87) (end 140.81 88.726514) (width 0.25) (layer "F.Cu") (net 3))
 (segment (start 159.315 100.23) (end 158.73 100.23) (width 0.25) (layer "F.Cu") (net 3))
 (via (at 158.194442 99.694442) (size 0.6) (drill 0.3) (layers "F.Cu" "B.Cu") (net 3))
 (via (at 137 93.5) (size 0.6) (drill 0.3) (layers "F.Cu" "B.Cu") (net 3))
 (via (at 157.310558 98.810558) (size 0.6) (drill 0.3) (layers "F.Cu" "B.Cu") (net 3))
 (via (at 139 91) (size 0.6) (drill 0.3) (layers "F.Cu" "B.Cu") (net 3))
 (segment (start 137 93.5) (end 137 93) (width 0.25) (layer "B.Cu") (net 3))
 (segment (start 158.194442 99.694442) (end 157.310558 98.810558) (width 0.25) (layer "B.Cu") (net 3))
 (segment (start 137 93) (end 139 91) (width 0.25) (layer "B.Cu") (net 3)))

